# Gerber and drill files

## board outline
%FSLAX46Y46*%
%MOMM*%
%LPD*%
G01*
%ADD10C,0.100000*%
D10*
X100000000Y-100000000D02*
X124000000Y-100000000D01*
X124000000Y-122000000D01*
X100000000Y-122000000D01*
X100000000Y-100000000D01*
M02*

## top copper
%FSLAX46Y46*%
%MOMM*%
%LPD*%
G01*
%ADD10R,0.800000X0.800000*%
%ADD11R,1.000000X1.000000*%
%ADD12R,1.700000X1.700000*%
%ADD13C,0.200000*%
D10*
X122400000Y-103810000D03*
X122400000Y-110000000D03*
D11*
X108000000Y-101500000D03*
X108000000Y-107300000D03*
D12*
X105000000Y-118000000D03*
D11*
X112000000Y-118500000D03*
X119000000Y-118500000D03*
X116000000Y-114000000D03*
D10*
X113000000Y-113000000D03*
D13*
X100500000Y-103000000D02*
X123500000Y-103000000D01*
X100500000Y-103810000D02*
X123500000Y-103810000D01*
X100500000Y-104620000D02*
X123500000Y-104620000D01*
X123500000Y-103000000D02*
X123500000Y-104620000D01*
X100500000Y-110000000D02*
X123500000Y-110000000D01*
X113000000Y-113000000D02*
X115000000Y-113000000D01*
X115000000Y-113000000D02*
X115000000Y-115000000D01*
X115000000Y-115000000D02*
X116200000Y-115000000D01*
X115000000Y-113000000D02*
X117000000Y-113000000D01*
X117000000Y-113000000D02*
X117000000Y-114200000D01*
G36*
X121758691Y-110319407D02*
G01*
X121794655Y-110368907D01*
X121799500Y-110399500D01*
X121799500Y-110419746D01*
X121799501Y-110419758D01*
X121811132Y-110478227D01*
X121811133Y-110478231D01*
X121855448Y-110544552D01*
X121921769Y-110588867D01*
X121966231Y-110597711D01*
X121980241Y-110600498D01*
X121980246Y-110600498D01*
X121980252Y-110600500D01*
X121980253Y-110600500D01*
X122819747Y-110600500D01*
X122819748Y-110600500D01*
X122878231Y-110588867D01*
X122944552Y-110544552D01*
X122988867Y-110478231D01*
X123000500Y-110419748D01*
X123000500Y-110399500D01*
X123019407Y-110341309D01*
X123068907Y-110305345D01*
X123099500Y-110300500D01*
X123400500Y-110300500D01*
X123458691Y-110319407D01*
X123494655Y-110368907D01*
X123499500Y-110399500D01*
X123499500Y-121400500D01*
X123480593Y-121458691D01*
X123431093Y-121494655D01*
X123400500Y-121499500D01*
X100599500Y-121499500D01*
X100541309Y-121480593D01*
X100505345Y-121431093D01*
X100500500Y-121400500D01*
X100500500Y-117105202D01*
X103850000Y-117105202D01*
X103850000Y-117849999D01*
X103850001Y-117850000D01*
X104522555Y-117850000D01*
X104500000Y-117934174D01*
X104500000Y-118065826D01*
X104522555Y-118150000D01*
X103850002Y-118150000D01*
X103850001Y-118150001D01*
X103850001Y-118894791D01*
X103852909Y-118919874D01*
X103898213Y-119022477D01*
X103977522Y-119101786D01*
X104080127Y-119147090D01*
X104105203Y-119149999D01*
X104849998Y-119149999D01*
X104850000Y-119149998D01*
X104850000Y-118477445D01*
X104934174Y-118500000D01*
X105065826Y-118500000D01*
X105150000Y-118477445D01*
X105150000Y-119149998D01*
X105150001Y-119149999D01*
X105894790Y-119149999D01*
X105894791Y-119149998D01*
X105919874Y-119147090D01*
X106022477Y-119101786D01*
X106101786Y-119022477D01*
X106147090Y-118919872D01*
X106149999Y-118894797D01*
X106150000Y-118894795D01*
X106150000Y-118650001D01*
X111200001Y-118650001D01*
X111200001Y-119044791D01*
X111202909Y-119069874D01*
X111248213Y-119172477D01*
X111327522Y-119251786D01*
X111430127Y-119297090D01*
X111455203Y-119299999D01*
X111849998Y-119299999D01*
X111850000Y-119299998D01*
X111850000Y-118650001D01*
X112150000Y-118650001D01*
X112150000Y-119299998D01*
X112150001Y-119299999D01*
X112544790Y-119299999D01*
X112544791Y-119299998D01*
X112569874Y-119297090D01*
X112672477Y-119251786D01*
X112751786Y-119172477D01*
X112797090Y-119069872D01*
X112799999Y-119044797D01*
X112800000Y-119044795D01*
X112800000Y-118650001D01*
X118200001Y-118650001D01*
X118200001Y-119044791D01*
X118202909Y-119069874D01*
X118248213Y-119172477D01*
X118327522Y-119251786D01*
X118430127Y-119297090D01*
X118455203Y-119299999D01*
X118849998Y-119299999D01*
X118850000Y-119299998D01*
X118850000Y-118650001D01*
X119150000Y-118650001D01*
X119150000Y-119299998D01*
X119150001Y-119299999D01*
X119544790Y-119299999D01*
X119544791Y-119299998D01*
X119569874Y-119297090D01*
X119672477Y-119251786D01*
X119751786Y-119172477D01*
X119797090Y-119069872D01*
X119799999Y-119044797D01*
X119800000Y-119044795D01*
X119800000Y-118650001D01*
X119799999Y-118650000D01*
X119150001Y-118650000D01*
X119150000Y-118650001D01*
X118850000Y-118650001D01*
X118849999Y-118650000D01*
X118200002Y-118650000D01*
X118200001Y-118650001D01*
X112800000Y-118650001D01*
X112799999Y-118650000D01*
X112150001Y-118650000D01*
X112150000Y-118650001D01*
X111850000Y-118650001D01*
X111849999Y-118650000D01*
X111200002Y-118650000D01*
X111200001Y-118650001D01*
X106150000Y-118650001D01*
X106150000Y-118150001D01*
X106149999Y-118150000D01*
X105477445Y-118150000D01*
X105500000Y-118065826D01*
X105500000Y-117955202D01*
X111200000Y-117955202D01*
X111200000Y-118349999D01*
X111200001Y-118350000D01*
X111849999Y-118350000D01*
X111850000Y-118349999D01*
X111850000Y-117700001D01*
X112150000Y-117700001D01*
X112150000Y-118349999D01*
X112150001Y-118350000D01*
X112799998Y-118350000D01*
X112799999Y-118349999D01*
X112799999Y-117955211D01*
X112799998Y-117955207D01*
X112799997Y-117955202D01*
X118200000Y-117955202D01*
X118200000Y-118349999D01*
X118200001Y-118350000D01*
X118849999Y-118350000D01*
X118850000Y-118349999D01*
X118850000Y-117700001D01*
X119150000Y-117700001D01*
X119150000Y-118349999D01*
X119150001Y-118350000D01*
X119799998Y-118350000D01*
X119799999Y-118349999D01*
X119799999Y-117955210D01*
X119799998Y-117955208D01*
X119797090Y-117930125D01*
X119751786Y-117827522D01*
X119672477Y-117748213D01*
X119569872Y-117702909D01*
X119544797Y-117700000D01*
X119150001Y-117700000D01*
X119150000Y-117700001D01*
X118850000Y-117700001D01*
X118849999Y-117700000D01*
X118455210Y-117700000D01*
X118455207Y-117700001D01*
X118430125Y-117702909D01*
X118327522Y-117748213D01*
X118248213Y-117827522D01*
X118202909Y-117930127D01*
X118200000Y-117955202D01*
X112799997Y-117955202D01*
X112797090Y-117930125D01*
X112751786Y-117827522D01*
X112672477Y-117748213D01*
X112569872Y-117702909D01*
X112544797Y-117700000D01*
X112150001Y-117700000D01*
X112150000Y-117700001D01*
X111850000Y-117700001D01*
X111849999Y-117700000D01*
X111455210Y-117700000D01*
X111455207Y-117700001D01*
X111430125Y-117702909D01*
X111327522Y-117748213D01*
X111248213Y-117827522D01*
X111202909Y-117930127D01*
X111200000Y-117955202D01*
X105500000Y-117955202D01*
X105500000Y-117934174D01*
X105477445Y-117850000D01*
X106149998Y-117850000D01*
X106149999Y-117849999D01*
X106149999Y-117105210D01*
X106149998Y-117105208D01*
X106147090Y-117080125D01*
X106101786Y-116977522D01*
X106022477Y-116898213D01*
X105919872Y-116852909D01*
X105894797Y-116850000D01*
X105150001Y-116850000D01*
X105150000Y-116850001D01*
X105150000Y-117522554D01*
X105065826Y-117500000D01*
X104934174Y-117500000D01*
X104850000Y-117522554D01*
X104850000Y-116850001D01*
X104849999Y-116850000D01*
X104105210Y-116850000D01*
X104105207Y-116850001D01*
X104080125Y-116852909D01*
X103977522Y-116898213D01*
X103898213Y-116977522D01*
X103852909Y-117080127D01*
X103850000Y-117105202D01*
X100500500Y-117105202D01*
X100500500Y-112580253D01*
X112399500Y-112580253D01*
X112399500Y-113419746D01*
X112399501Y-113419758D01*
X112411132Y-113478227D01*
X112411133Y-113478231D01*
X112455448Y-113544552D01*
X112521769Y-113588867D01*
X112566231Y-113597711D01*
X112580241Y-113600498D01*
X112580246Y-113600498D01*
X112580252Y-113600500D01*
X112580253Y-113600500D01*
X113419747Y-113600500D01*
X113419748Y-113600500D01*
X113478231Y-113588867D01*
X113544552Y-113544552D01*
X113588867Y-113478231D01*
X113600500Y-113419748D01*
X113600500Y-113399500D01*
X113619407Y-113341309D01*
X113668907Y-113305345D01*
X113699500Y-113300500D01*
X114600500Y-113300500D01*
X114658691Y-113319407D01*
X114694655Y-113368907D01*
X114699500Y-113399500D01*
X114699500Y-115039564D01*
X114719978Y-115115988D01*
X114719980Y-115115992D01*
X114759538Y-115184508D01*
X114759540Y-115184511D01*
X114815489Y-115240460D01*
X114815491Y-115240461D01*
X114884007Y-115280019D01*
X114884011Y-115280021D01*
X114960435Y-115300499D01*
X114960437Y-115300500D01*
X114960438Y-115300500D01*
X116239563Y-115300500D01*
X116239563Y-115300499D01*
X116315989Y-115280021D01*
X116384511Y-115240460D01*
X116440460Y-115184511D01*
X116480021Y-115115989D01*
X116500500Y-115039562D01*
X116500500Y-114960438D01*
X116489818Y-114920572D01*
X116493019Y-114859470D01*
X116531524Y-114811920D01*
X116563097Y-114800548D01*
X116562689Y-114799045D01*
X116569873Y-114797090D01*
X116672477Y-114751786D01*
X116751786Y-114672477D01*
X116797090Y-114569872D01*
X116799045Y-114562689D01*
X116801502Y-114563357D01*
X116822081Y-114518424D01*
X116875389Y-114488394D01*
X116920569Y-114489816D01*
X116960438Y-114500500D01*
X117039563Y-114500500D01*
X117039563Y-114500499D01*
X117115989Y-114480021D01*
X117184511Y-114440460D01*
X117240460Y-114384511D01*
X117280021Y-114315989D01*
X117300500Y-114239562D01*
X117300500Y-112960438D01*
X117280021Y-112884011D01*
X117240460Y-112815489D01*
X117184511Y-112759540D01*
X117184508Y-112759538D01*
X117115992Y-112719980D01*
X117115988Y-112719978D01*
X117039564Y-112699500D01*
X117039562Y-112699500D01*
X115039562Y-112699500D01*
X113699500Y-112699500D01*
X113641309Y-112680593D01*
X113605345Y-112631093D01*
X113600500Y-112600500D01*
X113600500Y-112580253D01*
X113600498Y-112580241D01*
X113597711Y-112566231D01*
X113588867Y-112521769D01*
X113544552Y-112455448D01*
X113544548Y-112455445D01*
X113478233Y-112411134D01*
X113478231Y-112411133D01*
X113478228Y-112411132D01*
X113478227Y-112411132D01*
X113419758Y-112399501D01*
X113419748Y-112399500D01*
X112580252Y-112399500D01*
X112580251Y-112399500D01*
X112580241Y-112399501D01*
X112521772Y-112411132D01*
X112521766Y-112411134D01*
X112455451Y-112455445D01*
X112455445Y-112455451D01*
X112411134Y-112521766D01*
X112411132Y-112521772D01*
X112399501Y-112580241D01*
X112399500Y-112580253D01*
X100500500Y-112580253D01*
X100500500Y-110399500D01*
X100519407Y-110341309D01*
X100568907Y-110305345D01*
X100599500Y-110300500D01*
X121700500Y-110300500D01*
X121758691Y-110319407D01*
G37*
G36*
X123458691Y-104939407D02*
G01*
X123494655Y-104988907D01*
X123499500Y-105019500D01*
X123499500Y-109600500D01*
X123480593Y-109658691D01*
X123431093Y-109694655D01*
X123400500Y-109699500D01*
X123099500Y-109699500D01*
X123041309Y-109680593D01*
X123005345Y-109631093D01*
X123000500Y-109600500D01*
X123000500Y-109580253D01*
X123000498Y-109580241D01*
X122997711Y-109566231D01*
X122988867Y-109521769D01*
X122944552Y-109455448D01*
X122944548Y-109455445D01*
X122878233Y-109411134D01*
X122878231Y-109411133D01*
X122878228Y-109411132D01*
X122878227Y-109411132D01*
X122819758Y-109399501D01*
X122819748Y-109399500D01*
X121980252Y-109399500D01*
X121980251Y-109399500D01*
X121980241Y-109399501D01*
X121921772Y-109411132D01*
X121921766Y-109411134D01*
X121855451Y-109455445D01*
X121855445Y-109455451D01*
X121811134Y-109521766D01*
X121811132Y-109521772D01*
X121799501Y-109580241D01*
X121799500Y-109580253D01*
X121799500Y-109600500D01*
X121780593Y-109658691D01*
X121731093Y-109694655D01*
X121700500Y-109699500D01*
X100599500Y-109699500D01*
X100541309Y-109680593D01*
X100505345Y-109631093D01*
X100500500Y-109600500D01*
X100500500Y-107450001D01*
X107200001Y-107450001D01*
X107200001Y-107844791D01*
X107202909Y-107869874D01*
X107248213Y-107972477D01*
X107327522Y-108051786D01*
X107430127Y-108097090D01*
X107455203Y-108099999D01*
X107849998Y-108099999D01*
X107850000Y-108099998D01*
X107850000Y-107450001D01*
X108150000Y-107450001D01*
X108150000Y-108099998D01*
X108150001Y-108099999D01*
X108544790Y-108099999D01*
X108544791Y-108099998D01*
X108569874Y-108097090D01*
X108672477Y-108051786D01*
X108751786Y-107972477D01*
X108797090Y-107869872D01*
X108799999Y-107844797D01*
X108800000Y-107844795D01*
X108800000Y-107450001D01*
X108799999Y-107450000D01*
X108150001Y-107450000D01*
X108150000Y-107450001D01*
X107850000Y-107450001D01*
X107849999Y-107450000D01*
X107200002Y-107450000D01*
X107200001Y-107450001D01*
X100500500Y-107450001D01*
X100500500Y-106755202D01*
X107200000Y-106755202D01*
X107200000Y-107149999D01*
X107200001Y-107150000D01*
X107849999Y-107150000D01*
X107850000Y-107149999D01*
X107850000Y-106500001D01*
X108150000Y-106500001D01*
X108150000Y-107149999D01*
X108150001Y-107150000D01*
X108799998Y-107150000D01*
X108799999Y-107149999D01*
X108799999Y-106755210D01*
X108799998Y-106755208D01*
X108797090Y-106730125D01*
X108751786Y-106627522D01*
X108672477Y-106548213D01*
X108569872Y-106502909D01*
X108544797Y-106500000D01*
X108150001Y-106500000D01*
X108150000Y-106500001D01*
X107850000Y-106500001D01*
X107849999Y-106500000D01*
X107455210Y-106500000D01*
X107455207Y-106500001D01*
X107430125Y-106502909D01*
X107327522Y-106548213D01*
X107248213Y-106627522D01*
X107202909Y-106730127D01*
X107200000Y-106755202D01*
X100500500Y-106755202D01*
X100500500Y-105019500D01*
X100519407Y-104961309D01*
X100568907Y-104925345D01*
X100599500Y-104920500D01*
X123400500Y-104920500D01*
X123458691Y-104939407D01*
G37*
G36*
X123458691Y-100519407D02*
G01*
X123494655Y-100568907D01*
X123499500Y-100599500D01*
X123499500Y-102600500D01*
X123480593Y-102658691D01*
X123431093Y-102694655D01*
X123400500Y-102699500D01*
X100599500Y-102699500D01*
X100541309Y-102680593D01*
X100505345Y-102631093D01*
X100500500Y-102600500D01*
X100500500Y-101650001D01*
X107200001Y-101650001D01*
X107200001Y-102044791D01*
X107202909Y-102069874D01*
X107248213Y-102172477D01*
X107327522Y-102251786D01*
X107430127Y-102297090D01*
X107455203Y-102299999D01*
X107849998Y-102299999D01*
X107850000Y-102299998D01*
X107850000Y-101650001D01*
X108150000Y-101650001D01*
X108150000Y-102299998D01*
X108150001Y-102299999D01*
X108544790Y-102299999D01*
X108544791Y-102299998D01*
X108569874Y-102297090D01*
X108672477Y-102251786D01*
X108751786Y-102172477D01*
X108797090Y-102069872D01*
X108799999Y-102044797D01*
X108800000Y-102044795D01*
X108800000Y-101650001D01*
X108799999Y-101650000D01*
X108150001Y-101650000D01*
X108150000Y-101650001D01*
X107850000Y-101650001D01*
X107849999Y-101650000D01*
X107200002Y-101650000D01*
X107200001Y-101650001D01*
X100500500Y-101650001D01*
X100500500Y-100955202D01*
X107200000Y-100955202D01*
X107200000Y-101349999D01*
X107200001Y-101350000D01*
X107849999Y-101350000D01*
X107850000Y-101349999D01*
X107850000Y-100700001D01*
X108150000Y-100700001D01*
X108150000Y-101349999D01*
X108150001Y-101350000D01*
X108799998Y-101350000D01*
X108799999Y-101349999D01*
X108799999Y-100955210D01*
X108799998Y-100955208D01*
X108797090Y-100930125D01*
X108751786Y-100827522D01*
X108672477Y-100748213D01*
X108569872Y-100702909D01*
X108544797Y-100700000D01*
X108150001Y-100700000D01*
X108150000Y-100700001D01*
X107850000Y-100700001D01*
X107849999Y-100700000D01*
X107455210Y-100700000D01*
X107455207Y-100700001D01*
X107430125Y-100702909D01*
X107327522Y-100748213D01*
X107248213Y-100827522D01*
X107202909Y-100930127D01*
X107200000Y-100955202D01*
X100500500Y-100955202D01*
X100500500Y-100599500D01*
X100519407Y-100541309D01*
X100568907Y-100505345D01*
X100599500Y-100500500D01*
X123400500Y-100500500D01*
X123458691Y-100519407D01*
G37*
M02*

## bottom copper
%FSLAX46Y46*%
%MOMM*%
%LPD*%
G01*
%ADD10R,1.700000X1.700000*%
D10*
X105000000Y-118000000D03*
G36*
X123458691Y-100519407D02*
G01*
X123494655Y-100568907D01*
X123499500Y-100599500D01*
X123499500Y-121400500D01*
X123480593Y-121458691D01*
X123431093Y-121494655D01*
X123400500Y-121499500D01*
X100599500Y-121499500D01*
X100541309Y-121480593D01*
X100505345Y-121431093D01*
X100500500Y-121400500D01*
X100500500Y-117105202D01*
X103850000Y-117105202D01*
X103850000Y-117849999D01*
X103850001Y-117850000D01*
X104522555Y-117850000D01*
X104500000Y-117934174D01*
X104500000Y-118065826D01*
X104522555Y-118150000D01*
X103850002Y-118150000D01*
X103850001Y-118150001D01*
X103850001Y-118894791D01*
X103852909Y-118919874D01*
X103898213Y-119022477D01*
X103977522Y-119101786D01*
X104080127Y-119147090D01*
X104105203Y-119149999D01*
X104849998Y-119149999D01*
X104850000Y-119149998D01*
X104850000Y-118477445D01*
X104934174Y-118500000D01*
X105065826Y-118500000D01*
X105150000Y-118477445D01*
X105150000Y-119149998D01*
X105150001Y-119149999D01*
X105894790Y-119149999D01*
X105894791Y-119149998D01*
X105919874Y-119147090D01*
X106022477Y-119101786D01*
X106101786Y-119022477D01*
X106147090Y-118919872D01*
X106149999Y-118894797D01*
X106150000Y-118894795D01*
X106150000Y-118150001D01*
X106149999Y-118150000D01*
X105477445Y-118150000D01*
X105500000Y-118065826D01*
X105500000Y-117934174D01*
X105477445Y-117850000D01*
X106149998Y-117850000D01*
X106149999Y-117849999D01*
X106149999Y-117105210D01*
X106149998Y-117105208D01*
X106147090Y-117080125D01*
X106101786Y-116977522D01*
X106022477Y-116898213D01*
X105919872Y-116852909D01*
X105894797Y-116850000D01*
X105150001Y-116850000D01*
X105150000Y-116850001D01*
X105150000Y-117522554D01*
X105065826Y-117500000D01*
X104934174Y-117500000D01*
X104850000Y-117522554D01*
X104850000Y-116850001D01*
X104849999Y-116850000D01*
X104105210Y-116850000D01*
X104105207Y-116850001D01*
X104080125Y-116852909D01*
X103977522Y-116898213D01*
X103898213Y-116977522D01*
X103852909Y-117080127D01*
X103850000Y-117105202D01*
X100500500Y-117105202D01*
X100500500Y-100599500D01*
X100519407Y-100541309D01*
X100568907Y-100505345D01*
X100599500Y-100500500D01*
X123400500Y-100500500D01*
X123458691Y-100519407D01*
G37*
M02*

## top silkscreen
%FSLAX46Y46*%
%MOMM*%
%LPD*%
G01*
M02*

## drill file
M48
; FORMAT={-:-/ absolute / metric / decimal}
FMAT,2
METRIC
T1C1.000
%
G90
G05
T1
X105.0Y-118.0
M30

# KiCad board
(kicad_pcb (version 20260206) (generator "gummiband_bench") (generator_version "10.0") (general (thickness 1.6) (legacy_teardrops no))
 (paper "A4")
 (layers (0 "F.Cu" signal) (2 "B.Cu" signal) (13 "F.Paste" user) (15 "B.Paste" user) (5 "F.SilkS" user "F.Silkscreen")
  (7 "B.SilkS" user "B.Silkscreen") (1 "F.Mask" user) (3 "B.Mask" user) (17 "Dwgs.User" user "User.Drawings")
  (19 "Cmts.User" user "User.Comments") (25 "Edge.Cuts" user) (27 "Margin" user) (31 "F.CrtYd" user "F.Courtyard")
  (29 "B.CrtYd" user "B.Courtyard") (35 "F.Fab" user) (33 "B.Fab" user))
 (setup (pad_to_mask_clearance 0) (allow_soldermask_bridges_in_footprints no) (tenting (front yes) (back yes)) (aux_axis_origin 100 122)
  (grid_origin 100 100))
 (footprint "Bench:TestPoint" (layer "F.Cu") (at 122.4 103.81)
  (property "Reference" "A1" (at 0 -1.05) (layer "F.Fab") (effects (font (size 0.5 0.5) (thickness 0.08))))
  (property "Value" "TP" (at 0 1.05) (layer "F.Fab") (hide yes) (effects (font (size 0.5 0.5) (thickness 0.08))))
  (pad "1" smd rect (at 0 0) (size 0.8 0.8) (layers "F.Cu" "F.Mask" "F.Paste") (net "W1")))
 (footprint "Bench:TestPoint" (layer "F.Cu") (at 122.4 110)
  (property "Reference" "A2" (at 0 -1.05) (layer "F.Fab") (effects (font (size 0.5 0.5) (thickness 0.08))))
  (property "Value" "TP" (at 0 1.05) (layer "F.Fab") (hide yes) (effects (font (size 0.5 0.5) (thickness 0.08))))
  (pad "1" smd rect (at 0 0) (size 0.8 0.8) (layers "F.Cu" "F.Mask" "F.Paste") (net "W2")))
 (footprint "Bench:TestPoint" (layer "F.Cu") (at 108 101.5)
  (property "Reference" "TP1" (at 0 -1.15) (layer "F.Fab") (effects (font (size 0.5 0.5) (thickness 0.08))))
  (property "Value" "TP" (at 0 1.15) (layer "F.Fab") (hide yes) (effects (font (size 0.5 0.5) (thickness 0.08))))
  (pad "1" smd rect (at 0 0) (size 1 1) (layers "F.Cu" "F.Mask" "F.Paste") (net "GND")))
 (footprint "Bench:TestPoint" (layer "F.Cu") (at 108 107.3)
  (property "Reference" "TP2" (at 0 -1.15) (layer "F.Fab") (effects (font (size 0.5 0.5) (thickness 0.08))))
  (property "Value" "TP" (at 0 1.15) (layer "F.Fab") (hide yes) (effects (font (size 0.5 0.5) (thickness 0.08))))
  (pad "1" smd rect (at 0 0) (size 1 1) (layers "F.Cu" "F.Mask" "F.Paste") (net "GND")))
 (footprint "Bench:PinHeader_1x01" (layer "F.Cu") (at 105 118)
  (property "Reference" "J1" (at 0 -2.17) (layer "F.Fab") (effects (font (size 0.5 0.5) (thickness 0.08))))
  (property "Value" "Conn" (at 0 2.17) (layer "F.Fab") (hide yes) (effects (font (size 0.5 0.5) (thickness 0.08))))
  (pad "1" thru_hole rect (at 0 0) (size 1.7 1.7) (drill 1) (layers "*.Cu" "*.Mask") (remove_unused_layers no) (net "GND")))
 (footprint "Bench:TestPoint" (layer "F.Cu") (at 112 118.5)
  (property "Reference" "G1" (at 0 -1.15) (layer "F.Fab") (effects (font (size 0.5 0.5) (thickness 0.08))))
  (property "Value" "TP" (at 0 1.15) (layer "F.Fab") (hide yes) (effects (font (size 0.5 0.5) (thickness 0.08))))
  (pad "1" smd rect (at 0 0) (size 1 1) (layers "F.Cu" "F.Mask" "F.Paste") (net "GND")))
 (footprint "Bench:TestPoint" (layer "F.Cu") (at 119 118.5)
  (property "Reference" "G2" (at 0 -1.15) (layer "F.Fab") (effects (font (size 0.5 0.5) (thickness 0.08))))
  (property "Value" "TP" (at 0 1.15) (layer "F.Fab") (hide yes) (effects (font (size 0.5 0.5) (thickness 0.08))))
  (pad "1" smd rect (at 0 0) (size 1 1) (layers "F.Cu" "F.Mask" "F.Paste") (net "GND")))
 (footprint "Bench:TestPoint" (layer "F.Cu") (at 116 114)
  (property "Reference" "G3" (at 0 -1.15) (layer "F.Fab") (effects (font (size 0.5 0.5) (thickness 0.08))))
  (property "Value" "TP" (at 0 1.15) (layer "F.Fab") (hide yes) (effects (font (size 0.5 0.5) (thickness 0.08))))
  (pad "1" smd rect (at 0 0) (size 1 1) (layers "F.Cu" "F.Mask" "F.Paste") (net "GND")))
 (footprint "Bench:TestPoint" (layer "F.Cu") (at 113 113)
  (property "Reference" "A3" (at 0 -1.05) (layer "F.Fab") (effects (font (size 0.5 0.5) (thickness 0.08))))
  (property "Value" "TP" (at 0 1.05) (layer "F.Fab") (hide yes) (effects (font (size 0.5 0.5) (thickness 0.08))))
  (pad "1" smd rect (at 0 0) (size 0.8 0.8) (layers "F.Cu" "F.Mask" "F.Paste") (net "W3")))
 (gr_rect (start 100 100) (end 124 122) (stroke (width 0.1) (type default)) (fill no) (layer "Edge.Cuts"))
 (segment (locked yes) (start 100.5 103) (end 123.5 103) (width 0.2) (layer "F.Cu") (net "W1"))
 (segment (locked yes) (start 100.5 103.81) (end 123.5 103.81) (width 0.2) (layer "F.Cu") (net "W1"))
 (segment (locked yes) (start 100.5 104.62) (end 123.5 104.62) (width 0.2) (layer "F.Cu") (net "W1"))
 (segment (locked yes) (start 123.5 103) (end 123.5 104.62) (width 0.2) (layer "F.Cu") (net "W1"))
 (segment (locked yes) (start 100.5 110) (end 123.5 110) (width 0.2) (layer "F.Cu") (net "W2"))
 (segment (locked yes) (start 113 113) (end 115 113) (width 0.2) (layer "F.Cu") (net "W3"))
 (segment (locked yes) (start 115 113) (end 115 115) (width 0.2) (layer "F.Cu") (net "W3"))
 (segment (locked yes) (start 115 115) (end 116.2 115) (width 0.2) (layer "F.Cu") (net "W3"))
 (segment (locked yes) (start 115 113) (end 117 113) (width 0.2) (layer "F.Cu") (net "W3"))
 (segment (locked yes) (start 117 113) (end 117 114.2) (width 0.2) (layer "F.Cu") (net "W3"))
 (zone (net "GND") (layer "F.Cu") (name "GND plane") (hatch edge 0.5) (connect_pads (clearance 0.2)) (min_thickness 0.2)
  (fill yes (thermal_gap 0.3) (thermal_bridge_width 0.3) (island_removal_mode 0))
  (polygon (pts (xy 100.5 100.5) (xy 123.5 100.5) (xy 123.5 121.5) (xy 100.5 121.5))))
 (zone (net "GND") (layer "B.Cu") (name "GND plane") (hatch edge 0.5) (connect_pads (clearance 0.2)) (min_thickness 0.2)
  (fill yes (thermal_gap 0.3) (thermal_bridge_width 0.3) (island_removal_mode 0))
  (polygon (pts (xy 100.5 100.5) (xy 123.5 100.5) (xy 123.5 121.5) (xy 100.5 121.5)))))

